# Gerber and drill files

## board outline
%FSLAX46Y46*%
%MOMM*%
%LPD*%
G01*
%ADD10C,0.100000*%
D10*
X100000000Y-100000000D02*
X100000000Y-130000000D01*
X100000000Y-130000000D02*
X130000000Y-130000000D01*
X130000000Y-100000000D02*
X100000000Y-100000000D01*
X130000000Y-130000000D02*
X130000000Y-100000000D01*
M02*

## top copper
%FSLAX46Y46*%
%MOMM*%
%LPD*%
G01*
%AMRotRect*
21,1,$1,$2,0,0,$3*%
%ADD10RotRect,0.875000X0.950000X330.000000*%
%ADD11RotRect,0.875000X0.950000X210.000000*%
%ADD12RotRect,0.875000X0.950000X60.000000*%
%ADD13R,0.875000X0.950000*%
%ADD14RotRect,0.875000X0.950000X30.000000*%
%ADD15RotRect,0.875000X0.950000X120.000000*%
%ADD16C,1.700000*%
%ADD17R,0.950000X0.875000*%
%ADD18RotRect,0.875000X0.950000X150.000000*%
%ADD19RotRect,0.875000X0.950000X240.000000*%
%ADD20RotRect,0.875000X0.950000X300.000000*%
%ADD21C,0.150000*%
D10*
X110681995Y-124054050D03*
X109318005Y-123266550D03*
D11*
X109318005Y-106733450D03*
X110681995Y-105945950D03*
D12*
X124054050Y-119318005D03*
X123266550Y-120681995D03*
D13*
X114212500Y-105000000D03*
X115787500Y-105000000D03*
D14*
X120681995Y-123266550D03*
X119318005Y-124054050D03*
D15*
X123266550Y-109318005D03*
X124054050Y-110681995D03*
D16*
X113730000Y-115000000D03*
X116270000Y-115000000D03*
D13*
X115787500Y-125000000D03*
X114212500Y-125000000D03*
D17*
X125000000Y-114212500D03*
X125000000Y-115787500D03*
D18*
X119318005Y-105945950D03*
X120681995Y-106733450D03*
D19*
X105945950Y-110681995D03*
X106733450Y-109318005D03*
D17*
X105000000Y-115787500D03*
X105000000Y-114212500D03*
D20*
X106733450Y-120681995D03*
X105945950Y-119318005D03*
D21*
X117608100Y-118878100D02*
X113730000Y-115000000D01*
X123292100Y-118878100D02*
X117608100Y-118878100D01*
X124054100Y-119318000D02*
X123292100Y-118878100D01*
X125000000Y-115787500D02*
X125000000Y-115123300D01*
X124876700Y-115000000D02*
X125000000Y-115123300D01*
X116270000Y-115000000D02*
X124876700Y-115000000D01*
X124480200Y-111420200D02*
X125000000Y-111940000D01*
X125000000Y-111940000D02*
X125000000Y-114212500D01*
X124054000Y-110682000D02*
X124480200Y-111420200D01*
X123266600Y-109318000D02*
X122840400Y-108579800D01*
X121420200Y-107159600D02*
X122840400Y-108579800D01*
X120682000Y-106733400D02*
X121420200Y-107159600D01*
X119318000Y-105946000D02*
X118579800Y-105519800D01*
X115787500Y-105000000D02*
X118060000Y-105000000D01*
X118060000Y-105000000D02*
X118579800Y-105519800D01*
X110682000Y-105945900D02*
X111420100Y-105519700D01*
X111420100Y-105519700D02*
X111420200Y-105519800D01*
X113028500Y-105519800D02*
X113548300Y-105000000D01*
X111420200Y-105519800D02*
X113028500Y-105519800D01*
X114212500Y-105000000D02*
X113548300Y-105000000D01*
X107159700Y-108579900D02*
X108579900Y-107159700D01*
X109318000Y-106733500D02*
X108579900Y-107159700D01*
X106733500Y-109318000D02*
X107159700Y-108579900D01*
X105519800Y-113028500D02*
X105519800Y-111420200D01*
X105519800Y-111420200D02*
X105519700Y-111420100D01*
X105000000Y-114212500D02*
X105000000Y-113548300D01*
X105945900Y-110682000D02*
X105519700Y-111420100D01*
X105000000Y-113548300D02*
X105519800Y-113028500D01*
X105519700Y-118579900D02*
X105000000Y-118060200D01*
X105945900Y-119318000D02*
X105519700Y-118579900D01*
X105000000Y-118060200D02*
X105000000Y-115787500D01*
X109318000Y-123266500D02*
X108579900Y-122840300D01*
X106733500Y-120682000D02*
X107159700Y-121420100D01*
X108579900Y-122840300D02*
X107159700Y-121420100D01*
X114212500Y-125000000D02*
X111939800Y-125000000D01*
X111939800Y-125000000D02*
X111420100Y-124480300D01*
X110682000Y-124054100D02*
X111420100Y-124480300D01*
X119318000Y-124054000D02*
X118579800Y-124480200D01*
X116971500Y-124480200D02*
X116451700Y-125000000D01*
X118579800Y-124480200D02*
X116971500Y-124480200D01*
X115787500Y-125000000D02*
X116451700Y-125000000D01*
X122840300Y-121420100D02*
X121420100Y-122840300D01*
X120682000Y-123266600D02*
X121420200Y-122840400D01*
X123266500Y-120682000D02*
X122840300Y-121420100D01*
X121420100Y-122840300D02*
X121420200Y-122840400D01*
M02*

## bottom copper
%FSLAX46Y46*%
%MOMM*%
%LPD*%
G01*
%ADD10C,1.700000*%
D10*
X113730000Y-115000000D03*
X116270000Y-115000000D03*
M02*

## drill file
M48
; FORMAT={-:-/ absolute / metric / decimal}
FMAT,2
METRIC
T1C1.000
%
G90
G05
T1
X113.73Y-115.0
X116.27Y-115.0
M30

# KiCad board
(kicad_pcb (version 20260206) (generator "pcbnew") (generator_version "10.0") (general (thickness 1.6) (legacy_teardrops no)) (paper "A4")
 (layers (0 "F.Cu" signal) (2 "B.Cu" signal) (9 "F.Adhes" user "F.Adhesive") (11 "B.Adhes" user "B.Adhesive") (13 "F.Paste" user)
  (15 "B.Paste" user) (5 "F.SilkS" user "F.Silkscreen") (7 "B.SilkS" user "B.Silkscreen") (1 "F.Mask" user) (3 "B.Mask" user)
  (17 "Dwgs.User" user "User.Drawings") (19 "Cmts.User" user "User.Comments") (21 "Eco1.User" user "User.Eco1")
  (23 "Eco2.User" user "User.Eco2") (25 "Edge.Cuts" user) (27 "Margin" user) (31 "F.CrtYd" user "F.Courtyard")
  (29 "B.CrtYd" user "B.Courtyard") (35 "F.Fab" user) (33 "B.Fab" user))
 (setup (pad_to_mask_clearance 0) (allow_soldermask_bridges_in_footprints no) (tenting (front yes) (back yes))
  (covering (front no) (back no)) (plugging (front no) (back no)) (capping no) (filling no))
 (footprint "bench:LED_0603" (layer "F.Cu") (at 110 123.6603 -30)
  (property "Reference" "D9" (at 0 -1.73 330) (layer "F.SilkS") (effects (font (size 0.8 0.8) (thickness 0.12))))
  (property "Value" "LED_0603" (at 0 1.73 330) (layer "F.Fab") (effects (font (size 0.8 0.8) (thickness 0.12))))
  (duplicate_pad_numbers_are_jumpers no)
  (pad "A" smd rect (at 0.7875 0 330) (size 0.875 0.95) (layers "F.Cu" "F.Mask" "F.Paste") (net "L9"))
  (pad "K" smd rect (at -0.7875 0 330) (size 0.875 0.95) (layers "F.Cu" "F.Mask" "F.Paste") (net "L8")))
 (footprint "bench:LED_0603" (layer "F.Cu") (at 110 106.3397 -150)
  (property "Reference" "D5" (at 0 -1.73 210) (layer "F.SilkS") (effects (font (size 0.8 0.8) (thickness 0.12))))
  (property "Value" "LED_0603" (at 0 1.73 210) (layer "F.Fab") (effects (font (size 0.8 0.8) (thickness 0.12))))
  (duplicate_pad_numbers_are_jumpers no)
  (pad "A" smd rect (at 0.7875 0 210) (size 0.875 0.95) (layers "F.Cu" "F.Mask" "F.Paste") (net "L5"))
  (pad "K" smd rect (at -0.7875 0 210) (size 0.875 0.95) (layers "F.Cu" "F.Mask" "F.Paste") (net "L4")))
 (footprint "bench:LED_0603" (layer "F.Cu") (at 123.6603 120 60)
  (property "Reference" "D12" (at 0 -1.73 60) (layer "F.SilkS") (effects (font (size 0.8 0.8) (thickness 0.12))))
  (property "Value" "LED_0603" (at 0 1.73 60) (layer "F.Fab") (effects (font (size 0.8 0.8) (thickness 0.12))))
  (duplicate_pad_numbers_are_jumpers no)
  (pad "A" smd rect (at 0.7875 0 60) (size 0.875 0.95) (layers "F.Cu" "F.Mask" "F.Paste") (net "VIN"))
  (pad "K" smd rect (at -0.7875 0 60) (size 0.875 0.95) (layers "F.Cu" "F.Mask" "F.Paste") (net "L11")))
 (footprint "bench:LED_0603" (layer "F.Cu") (at 115 105 180)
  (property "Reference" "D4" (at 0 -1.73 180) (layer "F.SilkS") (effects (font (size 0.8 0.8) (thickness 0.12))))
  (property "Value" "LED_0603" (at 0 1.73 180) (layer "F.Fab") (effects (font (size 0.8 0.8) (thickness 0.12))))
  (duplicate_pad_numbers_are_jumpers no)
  (pad "A" smd rect (at 0.7875 0 180) (size 0.875 0.95) (layers "F.Cu" "F.Mask" "F.Paste") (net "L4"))
  (pad "K" smd rect (at -0.7875 0 180) (size 0.875 0.95) (layers "F.Cu" "F.Mask" "F.Paste") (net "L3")))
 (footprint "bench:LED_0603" (layer "F.Cu") (at 120 123.6603 30)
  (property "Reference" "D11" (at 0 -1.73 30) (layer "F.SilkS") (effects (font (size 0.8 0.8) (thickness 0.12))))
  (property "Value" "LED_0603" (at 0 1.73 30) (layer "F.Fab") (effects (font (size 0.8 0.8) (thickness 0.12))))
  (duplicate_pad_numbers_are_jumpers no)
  (pad "A" smd rect (at 0.7875 0 30) (size 0.875 0.95) (layers "F.Cu" "F.Mask" "F.Paste") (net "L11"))
  (pad "K" smd rect (at -0.7875 0 30) (size 0.875 0.95) (layers "F.Cu" "F.Mask" "F.Paste") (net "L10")))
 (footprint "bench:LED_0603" (layer "F.Cu") (at 123.6603 110 120)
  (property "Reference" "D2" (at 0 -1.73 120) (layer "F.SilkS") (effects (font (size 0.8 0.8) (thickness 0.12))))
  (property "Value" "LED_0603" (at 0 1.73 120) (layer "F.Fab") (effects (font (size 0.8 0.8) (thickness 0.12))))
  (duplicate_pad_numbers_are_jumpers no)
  (pad "A" smd rect (at 0.7875 0 120) (size 0.875 0.95) (layers "F.Cu" "F.Mask" "F.Paste") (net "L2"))
  (pad "K" smd rect (at -0.7875 0 120) (size 0.875 0.95) (layers "F.Cu" "F.Mask" "F.Paste") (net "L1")))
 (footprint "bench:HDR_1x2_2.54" (layer "F.Cu") (at 113.73 115)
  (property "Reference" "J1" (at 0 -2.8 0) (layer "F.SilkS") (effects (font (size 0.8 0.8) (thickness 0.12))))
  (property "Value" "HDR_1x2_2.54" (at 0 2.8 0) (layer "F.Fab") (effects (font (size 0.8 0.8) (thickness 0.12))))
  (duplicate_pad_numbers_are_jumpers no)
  (pad "1" thru_hole circle (at 0 0) (size 1.7 1.7) (drill 1) (layers "*.Cu" "*.Mask") (remove_unused_layers no) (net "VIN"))
  (pad "2" thru_hole circle (at 2.54 0) (size 1.7 1.7) (drill 1) (layers "*.Cu" "*.Mask") (remove_unused_layers no) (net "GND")))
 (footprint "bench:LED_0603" (layer "F.Cu") (at 115 125)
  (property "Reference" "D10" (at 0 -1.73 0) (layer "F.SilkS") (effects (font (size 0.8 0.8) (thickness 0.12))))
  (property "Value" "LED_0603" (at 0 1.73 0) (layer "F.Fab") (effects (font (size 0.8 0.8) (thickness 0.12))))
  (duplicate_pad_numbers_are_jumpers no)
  (pad "A" smd rect (at 0.7875 0) (size 0.875 0.95) (layers "F.Cu" "F.Mask" "F.Paste") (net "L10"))
  (pad "K" smd rect (at -0.7875 0) (size 0.875 0.95) (layers "F.Cu" "F.Mask" "F.Paste") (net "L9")))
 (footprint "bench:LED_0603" (layer "F.Cu") (at 125 115 90)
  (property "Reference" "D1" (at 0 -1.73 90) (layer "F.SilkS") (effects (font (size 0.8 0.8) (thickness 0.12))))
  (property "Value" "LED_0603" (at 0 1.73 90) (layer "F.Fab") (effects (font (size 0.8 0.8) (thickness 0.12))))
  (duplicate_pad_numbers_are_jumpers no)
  (pad "A" smd rect (at 0.7875 0 90) (size 0.875 0.95) (layers "F.Cu" "F.Mask" "F.Paste") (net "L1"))
  (pad "K" smd rect (at -0.7875 0 90) (size 0.875 0.95) (layers "F.Cu" "F.Mask" "F.Paste") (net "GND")))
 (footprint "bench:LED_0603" (layer "F.Cu") (at 120 106.3397 150)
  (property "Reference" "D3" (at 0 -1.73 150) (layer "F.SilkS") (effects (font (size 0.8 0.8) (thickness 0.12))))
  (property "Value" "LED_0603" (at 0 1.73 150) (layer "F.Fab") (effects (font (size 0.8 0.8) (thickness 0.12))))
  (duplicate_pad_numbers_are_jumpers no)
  (pad "A" smd rect (at 0.7875 0 150) (size 0.875 0.95) (layers "F.Cu" "F.Mask" "F.Paste") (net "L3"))
  (pad "K" smd rect (at -0.7875 0 150) (size 0.875 0.95) (layers "F.Cu" "F.Mask" "F.Paste") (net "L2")))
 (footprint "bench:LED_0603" (layer "F.Cu") (at 106.3397 110 -120)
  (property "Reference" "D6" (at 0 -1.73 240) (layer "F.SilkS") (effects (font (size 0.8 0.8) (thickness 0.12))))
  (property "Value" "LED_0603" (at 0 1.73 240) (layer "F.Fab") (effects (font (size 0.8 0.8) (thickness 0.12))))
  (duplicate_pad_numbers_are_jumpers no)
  (pad "A" smd rect (at 0.7875 0 240) (size 0.875 0.95) (layers "F.Cu" "F.Mask" "F.Paste") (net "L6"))
  (pad "K" smd rect (at -0.7875 0 240) (size 0.875 0.95) (layers "F.Cu" "F.Mask" "F.Paste") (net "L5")))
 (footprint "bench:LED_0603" (layer "F.Cu") (at 105 115 -90)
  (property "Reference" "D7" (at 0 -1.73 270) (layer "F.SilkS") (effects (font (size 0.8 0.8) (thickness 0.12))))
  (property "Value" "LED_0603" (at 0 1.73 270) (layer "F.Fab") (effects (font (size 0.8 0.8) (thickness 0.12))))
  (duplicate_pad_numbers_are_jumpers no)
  (pad "A" smd rect (at 0.7875 0 270) (size 0.875 0.95) (layers "F.Cu" "F.Mask" "F.Paste") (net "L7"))
  (pad "K" smd rect (at -0.7875 0 270) (size 0.875 0.95) (layers "F.Cu" "F.Mask" "F.Paste") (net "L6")))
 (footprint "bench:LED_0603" (layer "F.Cu") (at 106.3397 120 -60)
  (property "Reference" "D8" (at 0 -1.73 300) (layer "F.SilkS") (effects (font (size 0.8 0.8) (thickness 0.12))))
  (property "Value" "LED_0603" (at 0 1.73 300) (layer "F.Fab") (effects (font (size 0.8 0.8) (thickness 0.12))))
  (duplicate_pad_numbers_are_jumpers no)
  (pad "A" smd rect (at 0.7875 0 300) (size 0.875 0.95) (layers "F.Cu" "F.Mask" "F.Paste") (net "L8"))
  (pad "K" smd rect (at -0.7875 0 300) (size 0.875 0.95) (layers "F.Cu" "F.Mask" "F.Paste") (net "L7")))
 (gr_line (start 100 100) (end 100 130) (stroke (width 0.1) (type solid)) (layer "Edge.Cuts"))
 (gr_line (start 100 130) (end 130 130) (stroke (width 0.1) (type solid)) (layer "Edge.Cuts"))
 (gr_line (start 130 100) (end 100 100) (stroke (width 0.1) (type solid)) (layer "Edge.Cuts"))
 (gr_line (start 130 130) (end 130 100) (stroke (width 0.1) (type solid)) (layer "Edge.Cuts"))
 (segment (start 117.6081 118.8781) (end 113.73 115) (width 0.15) (layer "F.Cu") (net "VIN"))
 (segment (start 123.2921 118.8781) (end 117.6081 118.8781) (width 0.15) (layer "F.Cu") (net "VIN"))
 (segment (start 124.0541 119.318) (end 123.2921 118.8781) (width 0.15) (layer "F.Cu") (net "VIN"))
 (segment (start 125 115.7875) (end 125 115.1233) (width 0.15) (layer "F.Cu") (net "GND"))
 (segment (start 124.8767 115) (end 125 115.1233) (width 0.15) (layer "F.Cu") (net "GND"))
 (segment (start 116.27 115) (end 124.8767 115) (width 0.15) (layer "F.Cu") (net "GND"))
 (segment (start 124.4802 111.4202) (end 125 111.94) (width 0.15) (layer "F.Cu") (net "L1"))
 (segment (start 125 111.94) (end 125 114.2125) (width 0.15) (layer "F.Cu") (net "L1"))
 (segment (start 124.054 110.682) (end 124.4802 111.4202) (width 0.15) (layer "F.Cu") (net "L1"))
 (segment (start 123.2666 109.318) (end 122.8404 108.5798) (width 0.15) (layer "F.Cu") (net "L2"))
 (segment (start 121.4202 107.1596) (end 122.8404 108.5798) (width 0.15) (layer "F.Cu") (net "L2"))
 (segment (start 120.682 106.7334) (end 121.4202 107.1596) (width 0.15) (layer "F.Cu") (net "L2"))
 (segment (start 119.318 105.946) (end 118.5798 105.5198) (width 0.15) (layer "F.Cu") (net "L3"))
 (segment (start 115.7875 105) (end 118.06 105) (width 0.15) (layer "F.Cu") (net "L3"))
 (segment (start 118.06 105) (end 118.5798 105.5198) (width 0.15) (layer "F.Cu") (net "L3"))
 (segment (start 110.682 105.9459) (end 111.4201 105.5197) (width 0.15) (layer "F.Cu") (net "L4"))
 (segment (start 111.4201 105.5197) (end 111.4202 105.5198) (width 0.15) (layer "F.Cu") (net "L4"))
 (segment (start 113.0285 105.5198) (end 113.5483 105) (width 0.15) (layer "F.Cu") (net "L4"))
 (segment (start 111.4202 105.5198) (end 113.0285 105.5198) (width 0.15) (layer "F.Cu") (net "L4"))
 (segment (start 114.2125 105) (end 113.5483 105) (width 0.15) (layer "F.Cu") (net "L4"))
 (segment (start 107.1597 108.5799) (end 108.5799 107.1597) (width 0.15) (layer "F.Cu") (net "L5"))
 (segment (start 109.318 106.7335) (end 108.5799 107.1597) (width 0.15) (layer "F.Cu") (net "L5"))
 (segment (start 106.7335 109.318) (end 107.1597 108.5799) (width 0.15) (layer "F.Cu") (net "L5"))
 (segment (start 105.5198 113.0285) (end 105.5198 111.4202) (width 0.15) (layer "F.Cu") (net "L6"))
 (segment (start 105.5198 111.4202) (end 105.5197 111.4201) (width 0.15) (layer "F.Cu") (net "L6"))
 (segment (start 105 114.2125) (end 105 113.5483) (width 0.15) (layer "F.Cu") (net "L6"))
 (segment (start 105.9459 110.682) (end 105.5197 111.4201) (width 0.15) (layer "F.Cu") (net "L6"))
 (segment (start 105 113.5483) (end 105.5198 113.0285) (width 0.15) (layer "F.Cu") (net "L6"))
 (segment (start 105.5197 118.5799) (end 105 118.0602) (width 0.15) (layer "F.Cu") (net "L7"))
 (segment (start 105.9459 119.318) (end 105.5197 118.5799) (width 0.15) (layer "F.Cu") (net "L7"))
 (segment (start 105 118.0602) (end 105 115.7875) (width 0.15) (layer "F.Cu") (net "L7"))
 (segment (start 109.318 123.2665) (end 108.5799 122.8403) (width 0.15) (layer "F.Cu") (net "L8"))
 (segment (start 106.7335 120.682) (end 107.1597 121.4201) (width 0.15) (layer "F.Cu") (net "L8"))
 (segment (start 108.5799 122.8403) (end 107.1597 121.4201) (width 0.15) (layer "F.Cu") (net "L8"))
 (segment (start 114.2125 125) (end 111.9398 125) (width 0.15) (layer "F.Cu") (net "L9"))
 (segment (start 111.9398 125) (end 111.4201 124.4803) (width 0.15) (layer "F.Cu") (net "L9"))
 (segment (start 110.682 124.0541) (end 111.4201 124.4803) (width 0.15) (layer "F.Cu") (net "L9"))
 (segment (start 119.318 124.054) (end 118.5798 124.4802) (width 0.15) (layer "F.Cu") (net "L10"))
 (segment (start 116.9715 124.4802) (end 116.4517 125) (width 0.15) (layer "F.Cu") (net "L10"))
 (segment (start 118.5798 124.4802) (end 116.9715 124.4802) (width 0.15) (layer "F.Cu") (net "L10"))
 (segment (start 115.7875 125) (end 116.4517 125) (width 0.15) (layer "F.Cu") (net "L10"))
 (segment (start 122.8403 121.4201) (end 121.4201 122.8403) (width 0.15) (layer "F.Cu") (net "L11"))
 (segment (start 120.682 123.2666) (end 121.4202 122.8404) (width 0.15) (layer "F.Cu") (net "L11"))
 (segment (start 123.2665 120.682) (end 122.8403 121.4201) (width 0.15) (layer "F.Cu") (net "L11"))
 (segment (start 121.4201 122.8403) (end 121.4202 122.8404) (width 0.15) (layer "F.Cu") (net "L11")))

